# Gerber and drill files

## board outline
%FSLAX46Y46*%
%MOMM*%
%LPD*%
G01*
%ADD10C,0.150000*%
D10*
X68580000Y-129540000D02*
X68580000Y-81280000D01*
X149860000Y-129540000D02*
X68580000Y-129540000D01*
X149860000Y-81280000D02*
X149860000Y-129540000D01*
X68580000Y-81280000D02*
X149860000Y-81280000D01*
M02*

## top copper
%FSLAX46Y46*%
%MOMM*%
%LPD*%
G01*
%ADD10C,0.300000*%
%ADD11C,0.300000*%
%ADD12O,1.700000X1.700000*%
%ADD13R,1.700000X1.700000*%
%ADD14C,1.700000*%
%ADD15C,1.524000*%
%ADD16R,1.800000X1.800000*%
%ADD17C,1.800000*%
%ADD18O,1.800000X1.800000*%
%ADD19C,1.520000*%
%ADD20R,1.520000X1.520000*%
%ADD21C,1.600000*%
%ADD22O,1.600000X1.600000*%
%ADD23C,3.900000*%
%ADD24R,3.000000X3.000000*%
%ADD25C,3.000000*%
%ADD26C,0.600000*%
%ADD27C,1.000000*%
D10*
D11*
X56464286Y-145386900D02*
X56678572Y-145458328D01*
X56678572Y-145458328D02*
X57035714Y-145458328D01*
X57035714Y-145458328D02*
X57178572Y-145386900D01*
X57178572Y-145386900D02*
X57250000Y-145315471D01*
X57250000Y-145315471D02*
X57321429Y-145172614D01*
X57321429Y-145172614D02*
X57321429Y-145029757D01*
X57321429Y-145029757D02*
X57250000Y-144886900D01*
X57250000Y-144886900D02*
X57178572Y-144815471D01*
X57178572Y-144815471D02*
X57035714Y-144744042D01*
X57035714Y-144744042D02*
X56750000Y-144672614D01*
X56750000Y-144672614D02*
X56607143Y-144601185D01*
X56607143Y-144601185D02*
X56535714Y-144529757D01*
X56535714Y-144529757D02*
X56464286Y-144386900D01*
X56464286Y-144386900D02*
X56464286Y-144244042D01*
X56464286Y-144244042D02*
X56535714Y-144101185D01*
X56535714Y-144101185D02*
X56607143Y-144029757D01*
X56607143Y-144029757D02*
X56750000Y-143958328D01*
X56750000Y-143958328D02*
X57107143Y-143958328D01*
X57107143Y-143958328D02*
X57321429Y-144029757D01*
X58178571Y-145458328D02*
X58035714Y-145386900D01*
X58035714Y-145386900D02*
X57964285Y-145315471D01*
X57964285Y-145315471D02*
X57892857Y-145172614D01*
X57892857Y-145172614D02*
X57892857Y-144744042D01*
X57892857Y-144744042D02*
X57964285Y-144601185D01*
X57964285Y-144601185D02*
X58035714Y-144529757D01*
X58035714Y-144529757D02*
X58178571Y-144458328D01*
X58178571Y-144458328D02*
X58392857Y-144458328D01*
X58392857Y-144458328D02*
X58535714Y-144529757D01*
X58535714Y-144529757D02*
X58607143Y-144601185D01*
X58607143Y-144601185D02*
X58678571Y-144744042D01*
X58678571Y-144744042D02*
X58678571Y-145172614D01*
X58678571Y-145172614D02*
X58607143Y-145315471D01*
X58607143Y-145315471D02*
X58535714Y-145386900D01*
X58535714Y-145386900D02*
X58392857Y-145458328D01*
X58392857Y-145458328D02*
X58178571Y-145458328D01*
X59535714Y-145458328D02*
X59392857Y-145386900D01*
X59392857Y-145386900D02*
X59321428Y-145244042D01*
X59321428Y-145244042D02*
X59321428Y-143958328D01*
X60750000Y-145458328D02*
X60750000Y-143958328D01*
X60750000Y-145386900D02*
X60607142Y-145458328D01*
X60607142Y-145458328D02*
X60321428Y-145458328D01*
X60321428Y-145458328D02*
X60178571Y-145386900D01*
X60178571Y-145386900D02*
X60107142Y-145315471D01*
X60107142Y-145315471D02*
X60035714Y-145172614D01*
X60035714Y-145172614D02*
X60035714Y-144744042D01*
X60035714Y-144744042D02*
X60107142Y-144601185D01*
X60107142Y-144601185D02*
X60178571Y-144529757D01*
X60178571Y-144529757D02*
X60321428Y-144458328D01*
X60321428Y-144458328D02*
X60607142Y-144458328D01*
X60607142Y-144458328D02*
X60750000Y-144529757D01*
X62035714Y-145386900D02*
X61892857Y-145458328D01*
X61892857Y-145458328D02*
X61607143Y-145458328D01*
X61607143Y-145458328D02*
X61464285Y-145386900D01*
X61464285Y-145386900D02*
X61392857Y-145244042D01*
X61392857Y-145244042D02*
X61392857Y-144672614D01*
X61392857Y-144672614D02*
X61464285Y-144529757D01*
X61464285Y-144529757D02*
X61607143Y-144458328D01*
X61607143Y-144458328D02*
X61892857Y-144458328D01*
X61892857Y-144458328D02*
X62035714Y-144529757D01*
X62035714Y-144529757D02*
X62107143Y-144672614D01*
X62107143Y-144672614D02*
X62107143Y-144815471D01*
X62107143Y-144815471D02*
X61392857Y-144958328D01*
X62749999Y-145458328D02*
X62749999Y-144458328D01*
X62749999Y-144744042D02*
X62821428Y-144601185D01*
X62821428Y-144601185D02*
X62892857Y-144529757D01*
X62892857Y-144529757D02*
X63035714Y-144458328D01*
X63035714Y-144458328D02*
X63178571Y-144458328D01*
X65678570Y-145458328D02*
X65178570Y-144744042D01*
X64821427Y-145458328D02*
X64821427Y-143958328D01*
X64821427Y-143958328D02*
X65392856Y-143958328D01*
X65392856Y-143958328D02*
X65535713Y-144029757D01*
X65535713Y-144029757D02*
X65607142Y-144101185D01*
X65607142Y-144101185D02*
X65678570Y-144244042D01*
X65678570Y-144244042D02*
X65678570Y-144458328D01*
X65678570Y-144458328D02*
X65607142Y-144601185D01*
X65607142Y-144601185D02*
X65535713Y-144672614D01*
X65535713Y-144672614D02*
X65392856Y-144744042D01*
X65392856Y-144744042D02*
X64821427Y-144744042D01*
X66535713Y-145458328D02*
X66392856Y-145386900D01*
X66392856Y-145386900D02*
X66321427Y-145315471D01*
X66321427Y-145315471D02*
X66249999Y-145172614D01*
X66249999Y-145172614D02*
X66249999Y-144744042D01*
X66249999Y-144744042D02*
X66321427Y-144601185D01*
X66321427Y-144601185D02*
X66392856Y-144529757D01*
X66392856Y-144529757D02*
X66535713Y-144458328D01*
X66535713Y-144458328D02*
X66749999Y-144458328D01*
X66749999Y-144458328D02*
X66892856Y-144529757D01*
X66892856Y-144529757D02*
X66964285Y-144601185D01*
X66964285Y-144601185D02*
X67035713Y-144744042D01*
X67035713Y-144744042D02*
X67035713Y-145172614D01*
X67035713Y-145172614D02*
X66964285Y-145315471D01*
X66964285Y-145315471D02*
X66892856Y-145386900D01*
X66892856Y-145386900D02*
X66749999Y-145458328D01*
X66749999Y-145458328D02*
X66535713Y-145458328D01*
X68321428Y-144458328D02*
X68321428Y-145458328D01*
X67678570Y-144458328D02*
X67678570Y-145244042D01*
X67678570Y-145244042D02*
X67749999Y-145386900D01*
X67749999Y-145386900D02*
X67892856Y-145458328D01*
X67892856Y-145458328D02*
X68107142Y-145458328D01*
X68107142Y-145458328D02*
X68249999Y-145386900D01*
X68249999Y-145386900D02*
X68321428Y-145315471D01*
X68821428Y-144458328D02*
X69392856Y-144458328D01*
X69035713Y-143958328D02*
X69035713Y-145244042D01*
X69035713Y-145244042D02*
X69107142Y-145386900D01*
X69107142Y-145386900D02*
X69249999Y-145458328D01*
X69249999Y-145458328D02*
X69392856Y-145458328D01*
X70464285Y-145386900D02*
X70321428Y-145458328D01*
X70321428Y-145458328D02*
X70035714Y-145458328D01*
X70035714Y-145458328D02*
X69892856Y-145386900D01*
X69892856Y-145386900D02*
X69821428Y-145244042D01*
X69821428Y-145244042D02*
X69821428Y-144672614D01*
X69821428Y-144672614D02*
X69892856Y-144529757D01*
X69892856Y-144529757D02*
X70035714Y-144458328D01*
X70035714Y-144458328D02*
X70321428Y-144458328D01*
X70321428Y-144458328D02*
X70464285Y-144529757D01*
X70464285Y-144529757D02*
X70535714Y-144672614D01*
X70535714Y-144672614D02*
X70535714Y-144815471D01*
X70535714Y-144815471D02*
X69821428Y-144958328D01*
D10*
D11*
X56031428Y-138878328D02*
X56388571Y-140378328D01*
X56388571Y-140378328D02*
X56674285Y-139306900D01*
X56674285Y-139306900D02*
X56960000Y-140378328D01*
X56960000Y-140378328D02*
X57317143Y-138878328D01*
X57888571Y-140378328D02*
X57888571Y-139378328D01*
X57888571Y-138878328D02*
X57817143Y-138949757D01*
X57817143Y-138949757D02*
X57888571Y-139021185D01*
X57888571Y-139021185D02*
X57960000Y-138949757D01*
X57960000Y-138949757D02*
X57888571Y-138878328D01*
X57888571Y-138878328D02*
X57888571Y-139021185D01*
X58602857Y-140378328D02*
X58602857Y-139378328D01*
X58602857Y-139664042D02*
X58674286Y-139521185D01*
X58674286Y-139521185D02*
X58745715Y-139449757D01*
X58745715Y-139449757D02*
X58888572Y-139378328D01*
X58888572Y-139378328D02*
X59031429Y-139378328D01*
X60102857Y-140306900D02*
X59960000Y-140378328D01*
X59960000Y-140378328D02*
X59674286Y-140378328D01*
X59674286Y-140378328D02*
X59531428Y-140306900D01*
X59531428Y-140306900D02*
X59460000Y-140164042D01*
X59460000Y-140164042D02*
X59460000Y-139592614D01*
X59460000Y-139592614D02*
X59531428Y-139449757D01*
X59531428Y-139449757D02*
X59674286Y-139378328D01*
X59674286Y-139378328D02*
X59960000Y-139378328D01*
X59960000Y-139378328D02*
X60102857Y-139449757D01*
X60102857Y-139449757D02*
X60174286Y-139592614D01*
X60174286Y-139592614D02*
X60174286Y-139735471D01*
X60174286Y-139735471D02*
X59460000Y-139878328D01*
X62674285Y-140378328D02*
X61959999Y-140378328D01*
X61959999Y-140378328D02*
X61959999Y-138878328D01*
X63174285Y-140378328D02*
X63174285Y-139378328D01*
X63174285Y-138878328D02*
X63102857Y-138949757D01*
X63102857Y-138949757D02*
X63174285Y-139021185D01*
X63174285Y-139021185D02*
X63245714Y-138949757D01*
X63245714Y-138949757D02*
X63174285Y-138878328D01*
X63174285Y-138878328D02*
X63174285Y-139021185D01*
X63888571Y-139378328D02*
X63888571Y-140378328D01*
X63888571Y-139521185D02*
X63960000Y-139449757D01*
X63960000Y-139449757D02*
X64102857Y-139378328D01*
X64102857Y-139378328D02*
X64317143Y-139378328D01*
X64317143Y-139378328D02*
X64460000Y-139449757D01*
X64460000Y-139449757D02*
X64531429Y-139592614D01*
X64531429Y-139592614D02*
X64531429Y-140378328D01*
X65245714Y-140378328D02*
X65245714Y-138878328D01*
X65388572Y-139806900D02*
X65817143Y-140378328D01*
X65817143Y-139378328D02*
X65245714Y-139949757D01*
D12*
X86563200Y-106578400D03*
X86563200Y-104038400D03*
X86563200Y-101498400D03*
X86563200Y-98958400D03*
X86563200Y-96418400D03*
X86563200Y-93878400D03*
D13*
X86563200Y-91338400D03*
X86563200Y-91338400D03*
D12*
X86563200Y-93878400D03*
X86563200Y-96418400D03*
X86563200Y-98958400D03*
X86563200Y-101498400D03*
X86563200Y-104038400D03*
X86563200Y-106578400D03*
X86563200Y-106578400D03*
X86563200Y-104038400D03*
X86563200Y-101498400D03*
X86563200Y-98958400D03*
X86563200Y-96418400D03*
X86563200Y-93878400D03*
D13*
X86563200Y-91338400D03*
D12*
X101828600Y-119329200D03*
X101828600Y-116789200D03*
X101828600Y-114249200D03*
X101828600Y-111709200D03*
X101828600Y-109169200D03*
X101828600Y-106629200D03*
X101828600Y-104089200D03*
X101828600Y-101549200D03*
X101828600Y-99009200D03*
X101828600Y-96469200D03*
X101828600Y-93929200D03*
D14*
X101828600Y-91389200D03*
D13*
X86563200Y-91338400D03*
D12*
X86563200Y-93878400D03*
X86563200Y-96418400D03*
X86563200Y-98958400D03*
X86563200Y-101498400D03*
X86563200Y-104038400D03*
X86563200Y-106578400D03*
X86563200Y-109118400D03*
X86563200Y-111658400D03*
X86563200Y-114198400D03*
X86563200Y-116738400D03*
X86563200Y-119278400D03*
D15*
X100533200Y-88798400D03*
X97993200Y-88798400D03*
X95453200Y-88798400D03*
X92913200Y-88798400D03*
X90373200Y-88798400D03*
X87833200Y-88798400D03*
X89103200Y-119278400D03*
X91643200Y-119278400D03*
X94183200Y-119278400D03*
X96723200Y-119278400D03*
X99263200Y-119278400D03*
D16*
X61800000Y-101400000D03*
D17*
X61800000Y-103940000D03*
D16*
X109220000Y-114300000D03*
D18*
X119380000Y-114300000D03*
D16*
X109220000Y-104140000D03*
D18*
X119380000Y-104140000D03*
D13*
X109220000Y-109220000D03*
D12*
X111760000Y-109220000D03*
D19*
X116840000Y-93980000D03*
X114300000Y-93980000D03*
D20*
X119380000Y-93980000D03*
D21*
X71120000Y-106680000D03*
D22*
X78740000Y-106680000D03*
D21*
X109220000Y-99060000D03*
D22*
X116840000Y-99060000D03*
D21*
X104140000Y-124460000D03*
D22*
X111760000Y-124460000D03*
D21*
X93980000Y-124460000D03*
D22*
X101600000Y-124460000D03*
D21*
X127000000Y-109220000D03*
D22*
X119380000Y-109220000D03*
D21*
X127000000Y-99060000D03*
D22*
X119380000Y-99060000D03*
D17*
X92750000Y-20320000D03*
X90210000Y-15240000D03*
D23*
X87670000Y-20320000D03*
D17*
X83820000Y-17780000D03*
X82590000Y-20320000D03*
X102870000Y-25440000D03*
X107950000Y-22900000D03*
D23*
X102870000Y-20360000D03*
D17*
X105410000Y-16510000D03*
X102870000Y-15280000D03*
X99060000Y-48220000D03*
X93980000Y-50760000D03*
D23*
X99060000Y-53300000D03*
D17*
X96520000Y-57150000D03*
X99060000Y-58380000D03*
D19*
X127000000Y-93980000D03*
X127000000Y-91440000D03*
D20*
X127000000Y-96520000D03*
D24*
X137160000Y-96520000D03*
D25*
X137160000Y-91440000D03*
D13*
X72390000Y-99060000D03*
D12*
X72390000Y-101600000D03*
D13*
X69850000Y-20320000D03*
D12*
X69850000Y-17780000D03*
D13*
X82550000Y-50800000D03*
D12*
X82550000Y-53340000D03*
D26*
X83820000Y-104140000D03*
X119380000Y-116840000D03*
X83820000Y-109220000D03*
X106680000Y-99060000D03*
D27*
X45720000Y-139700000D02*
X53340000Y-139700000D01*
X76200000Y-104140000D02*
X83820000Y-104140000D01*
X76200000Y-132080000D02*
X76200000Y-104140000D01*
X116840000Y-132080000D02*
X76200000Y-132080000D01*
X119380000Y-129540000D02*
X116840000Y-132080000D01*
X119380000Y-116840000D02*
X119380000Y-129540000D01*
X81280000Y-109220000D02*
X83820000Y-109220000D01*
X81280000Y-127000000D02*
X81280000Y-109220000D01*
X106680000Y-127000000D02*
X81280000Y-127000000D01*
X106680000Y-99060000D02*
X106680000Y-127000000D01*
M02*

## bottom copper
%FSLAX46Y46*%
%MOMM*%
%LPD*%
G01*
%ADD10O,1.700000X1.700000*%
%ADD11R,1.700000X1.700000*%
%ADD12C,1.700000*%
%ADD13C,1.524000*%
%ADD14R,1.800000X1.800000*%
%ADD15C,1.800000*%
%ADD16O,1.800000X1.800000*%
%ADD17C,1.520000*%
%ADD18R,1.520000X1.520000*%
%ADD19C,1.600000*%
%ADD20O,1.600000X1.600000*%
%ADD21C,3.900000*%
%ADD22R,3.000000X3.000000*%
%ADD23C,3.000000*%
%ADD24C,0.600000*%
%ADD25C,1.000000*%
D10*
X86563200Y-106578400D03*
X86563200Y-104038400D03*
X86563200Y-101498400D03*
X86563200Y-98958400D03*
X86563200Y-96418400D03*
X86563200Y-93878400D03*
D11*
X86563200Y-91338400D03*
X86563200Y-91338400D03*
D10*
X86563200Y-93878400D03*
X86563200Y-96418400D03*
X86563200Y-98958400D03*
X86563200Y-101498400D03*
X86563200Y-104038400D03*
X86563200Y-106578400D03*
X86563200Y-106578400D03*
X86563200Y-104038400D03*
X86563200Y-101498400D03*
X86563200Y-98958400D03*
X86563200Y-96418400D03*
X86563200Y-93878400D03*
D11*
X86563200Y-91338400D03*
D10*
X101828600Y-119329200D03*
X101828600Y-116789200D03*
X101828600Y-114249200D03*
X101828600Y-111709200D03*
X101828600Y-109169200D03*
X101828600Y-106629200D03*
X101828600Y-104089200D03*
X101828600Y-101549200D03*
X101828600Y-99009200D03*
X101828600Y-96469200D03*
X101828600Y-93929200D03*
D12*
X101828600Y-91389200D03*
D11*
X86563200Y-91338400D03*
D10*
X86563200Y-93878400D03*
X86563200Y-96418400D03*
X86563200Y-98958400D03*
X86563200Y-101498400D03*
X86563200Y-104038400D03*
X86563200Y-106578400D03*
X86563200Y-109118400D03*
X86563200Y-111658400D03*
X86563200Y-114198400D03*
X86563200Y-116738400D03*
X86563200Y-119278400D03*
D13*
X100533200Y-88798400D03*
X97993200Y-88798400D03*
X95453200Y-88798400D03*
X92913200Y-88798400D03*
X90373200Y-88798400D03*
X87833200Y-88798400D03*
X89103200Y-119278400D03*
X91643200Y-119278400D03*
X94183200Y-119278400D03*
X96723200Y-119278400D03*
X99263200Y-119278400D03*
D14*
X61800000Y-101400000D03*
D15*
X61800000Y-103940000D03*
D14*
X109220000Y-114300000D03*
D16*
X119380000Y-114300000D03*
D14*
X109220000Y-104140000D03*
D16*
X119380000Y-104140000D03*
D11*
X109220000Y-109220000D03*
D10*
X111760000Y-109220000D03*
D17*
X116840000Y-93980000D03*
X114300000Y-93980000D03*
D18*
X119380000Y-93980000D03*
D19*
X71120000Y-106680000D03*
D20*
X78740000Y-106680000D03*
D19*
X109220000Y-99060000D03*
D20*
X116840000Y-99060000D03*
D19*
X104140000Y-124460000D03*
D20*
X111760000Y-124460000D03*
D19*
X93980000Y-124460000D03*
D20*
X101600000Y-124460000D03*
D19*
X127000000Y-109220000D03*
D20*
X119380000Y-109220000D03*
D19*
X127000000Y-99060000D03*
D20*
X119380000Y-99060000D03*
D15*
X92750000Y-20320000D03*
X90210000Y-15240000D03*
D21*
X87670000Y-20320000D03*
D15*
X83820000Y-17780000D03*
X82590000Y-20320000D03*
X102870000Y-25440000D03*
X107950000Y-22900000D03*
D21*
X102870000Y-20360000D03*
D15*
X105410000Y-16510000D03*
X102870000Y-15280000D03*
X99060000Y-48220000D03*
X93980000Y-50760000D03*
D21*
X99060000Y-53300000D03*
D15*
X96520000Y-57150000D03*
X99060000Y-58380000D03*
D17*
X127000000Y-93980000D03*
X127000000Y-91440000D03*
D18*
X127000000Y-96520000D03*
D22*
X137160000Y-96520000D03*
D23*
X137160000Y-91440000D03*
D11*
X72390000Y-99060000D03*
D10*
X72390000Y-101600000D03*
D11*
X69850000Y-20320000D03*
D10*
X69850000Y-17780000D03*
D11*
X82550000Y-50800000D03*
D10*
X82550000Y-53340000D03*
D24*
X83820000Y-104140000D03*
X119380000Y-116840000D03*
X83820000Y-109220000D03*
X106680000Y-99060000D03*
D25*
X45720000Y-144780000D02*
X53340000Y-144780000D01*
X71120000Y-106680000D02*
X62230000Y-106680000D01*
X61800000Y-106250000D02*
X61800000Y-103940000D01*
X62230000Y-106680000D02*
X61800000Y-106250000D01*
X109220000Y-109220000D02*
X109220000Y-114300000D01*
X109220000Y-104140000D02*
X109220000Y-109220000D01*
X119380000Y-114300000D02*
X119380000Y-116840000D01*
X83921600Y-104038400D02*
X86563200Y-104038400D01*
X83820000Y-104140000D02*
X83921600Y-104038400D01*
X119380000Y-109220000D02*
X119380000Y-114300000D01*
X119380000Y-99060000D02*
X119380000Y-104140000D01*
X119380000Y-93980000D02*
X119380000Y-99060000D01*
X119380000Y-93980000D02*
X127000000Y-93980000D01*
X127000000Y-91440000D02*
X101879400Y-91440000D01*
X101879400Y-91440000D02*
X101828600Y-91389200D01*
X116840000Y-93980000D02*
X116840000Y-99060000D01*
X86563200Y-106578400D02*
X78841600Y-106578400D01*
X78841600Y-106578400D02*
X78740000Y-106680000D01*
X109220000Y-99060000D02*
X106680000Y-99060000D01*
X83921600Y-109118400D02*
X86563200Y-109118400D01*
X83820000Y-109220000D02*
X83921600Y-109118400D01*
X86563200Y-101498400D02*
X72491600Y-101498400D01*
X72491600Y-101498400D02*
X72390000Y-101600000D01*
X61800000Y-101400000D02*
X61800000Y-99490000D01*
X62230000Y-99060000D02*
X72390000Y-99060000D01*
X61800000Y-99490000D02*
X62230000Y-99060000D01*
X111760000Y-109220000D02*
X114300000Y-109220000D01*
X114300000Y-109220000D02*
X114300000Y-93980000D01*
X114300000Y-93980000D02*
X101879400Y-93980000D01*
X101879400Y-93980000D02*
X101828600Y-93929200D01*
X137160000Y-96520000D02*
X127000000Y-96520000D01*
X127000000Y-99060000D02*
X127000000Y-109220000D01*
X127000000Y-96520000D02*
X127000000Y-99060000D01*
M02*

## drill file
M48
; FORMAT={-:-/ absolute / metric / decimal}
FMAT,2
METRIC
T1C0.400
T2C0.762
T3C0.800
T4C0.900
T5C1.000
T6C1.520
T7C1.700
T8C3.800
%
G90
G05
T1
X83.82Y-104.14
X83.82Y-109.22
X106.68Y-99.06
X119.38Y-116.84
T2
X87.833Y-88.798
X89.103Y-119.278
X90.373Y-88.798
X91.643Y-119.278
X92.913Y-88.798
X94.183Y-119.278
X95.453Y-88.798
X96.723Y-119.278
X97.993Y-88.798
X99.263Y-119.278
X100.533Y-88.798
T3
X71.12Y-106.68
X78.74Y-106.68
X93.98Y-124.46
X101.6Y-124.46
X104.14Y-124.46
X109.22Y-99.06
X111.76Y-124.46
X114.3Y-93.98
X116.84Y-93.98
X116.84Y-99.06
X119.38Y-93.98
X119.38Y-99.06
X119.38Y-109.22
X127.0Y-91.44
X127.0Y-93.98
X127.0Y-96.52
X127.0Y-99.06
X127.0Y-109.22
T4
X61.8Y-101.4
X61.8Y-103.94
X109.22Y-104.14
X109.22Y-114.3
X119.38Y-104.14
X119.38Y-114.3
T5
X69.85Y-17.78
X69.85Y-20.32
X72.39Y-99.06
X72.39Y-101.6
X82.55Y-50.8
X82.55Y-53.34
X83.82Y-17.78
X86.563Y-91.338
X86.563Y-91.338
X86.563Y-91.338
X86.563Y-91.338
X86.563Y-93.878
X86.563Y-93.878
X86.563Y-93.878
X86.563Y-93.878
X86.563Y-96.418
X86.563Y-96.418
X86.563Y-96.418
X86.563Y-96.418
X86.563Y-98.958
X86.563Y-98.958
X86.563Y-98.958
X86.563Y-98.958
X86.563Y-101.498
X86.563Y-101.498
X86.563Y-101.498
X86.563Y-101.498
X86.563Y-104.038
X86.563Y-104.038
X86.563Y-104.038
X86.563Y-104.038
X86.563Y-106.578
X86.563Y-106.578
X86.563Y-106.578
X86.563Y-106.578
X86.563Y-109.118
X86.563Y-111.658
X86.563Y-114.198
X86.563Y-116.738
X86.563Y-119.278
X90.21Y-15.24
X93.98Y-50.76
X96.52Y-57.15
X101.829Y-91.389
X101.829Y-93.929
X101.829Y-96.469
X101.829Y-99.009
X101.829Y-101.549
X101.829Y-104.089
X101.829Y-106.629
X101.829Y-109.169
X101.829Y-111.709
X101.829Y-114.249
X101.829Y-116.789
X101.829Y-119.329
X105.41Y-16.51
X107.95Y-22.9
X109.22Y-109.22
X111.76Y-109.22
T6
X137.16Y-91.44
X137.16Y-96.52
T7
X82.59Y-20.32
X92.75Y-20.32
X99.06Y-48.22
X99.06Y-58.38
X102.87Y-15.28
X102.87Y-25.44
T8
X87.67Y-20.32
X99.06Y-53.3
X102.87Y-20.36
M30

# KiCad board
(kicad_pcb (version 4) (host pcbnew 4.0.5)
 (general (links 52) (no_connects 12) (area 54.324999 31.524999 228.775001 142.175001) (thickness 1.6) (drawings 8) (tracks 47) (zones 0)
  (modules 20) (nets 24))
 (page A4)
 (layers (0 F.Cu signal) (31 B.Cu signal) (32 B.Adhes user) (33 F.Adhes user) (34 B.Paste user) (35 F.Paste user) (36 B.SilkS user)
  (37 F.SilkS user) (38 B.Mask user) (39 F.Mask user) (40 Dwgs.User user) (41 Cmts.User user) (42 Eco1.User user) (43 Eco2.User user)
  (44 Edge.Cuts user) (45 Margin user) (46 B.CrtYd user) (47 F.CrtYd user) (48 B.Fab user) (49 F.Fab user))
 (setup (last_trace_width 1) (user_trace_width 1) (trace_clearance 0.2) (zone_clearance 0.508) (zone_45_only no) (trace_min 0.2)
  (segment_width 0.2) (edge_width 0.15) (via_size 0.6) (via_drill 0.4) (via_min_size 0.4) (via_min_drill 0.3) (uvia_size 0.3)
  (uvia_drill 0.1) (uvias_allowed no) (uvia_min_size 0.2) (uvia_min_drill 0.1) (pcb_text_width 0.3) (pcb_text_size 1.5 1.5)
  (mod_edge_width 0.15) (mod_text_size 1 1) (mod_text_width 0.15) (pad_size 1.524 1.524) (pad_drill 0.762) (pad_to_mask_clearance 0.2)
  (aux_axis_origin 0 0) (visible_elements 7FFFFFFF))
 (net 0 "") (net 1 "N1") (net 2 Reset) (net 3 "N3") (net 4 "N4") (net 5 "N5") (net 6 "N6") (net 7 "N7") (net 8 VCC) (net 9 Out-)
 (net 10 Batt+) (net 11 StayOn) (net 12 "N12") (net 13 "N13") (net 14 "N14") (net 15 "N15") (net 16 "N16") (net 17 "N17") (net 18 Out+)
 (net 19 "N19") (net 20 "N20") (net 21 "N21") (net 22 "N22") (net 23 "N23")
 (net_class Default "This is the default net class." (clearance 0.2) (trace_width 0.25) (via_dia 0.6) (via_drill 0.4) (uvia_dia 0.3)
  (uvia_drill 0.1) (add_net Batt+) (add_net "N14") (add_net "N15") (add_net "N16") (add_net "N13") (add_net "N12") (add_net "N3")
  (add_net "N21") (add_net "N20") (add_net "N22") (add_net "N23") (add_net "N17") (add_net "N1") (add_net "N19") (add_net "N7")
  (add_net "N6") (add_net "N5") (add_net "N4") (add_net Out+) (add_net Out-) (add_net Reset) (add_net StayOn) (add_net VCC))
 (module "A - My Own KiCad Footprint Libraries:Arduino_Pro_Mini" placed (layer F.Cu) (at 93.98 101.6)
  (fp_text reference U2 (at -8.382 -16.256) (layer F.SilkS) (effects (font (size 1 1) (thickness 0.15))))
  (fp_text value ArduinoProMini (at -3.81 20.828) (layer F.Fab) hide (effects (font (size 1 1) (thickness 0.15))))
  (pad 7 thru_hole oval (at -7.4168 4.9784) (size 1.7 1.7) (drill 1) (layers *.Mask B.Cu) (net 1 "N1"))
  (pad 6 thru_hole oval (at -7.4168 2.4384) (size 1.7 1.7) (drill 1) (layers *.Mask B.Cu) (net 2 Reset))
  (pad 5 thru_hole oval (at -7.4168 -0.1016) (size 1.7 1.7) (drill 1) (layers *.Mask B.Cu) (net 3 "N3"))
  (pad 4 thru_hole oval (at -7.4168 -2.6416) (size 1.7 1.7) (drill 1) (layers *.Mask B.Cu) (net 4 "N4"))
  (pad 3 thru_hole oval (at -7.4168 -5.1816) (size 1.7 1.7) (drill 1) (layers *.Mask B.Cu) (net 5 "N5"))
  (pad 2 thru_hole oval (at -7.4168 -7.7216) (size 1.7 1.7) (drill 1) (layers *.Mask B.Cu) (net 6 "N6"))
  (pad 1 thru_hole rect (at -7.4168 -10.2616) (size 1.7 1.7) (drill 1) (layers *.Mask B.Cu) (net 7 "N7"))
  (pad 1 thru_hole rect (at -7.4168 -10.2616) (size 1.7 1.7) (drill 1) (layers *.Mask B.Cu) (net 7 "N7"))
  (pad 2 thru_hole oval (at -7.4168 -7.7216) (size 1.7 1.7) (drill 1) (layers *.Mask B.Cu) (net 6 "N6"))
  (pad 3 thru_hole oval (at -7.4168 -5.1816) (size 1.7 1.7) (drill 1) (layers *.Mask B.Cu) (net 5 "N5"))
  (pad 4 thru_hole oval (at -7.4168 -2.6416) (size 1.7 1.7) (drill 1) (layers *.Mask B.Cu) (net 4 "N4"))
  (pad 5 thru_hole oval (at -7.4168 -0.1016) (size 1.7 1.7) (drill 1) (layers *.Mask B.Cu) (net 3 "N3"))
  (pad 6 thru_hole oval (at -7.4168 2.4384) (size 1.7 1.7) (drill 1) (layers *.Mask B.Cu) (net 2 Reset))
  (pad 7 thru_hole oval (at -7.4168 4.9784) (size 1.7 1.7) (drill 1) (layers *.Mask B.Cu) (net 1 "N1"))
  (pad 7 thru_hole oval (at -7.4168 4.9784) (size 1.7 1.7) (drill 1) (layers *.Mask B.Cu) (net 1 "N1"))
  (pad 6 thru_hole oval (at -7.4168 2.4384) (size 1.7 1.7) (drill 1) (layers *.Mask B.Cu) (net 2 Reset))
  (pad 5 thru_hole oval (at -7.4168 -0.1016) (size 1.7 1.7) (drill 1) (layers *.Mask B.Cu) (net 3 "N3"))
  (pad 4 thru_hole oval (at -7.4168 -2.6416) (size 1.7 1.7) (drill 1) (layers *.Mask B.Cu) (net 4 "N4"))
  (pad 3 thru_hole oval (at -7.4168 -5.1816) (size 1.7 1.7) (drill 1) (layers *.Mask B.Cu) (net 5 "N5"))
  (pad 2 thru_hole oval (at -7.4168 -7.7216) (size 1.7 1.7) (drill 1) (layers *.Mask B.Cu) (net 6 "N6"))
  (pad 1 thru_hole rect (at -7.4168 -10.2616) (size 1.7 1.7) (drill 1) (layers *.Mask B.Cu) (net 7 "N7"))
  (pad 18 thru_hole oval (at 7.8486 17.7292) (size 1.7 1.7) (drill 1) (layers *.Mask B.Cu))
  (pad 19 thru_hole oval (at 7.8486 15.1892) (size 1.7 1.7) (drill 1) (layers *.Mask B.Cu))
  (pad 20 thru_hole oval (at 7.8486 12.6492) (size 1.7 1.7) (drill 1) (layers *.Mask B.Cu))
  (pad 21 thru_hole oval (at 7.8486 10.1092) (size 1.7 1.7) (drill 1) (layers *.Mask B.Cu))
  (pad 22 thru_hole oval (at 7.8486 7.5692) (size 1.7 1.7) (drill 1) (layers *.Mask B.Cu))
  (pad 23 thru_hole oval (at 7.8486 5.0292) (size 1.7 1.7) (drill 1) (layers *.Mask B.Cu))
  (pad 24 thru_hole oval (at 7.8486 2.4892) (size 1.7 1.7) (drill 1) (layers *.Mask B.Cu))
  (pad 25 thru_hole oval (at 7.8486 -0.0508) (size 1.7 1.7) (drill 1) (layers *.Mask B.Cu))
  (pad 26 thru_hole oval (at 7.8486 -2.5908) (size 1.7 1.7) (drill 1) (layers *.Mask B.Cu) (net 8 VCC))
  (pad 27 thru_hole oval (at 7.8486 -5.1308) (size 1.7 1.7) (drill 1) (layers *.Mask B.Cu))
  (pad 28 thru_hole oval (at 7.8486 -7.6708) (size 1.7 1.7) (drill 1) (layers *.Mask B.Cu) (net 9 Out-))
  (pad 29 thru_hole circle (at 7.8486 -10.2108) (size 1.7 1.7) (drill 1) (layers *.Mask B.Cu) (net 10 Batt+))
  (pad 1 thru_hole rect (at -7.4168 -10.2616) (size 1.7 1.7) (drill 1) (layers *.Mask B.Cu) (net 7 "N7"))
  (pad 2 thru_hole oval (at -7.4168 -7.7216) (size 1.7 1.7) (drill 1) (layers *.Mask B.Cu) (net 6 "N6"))
  (pad 3 thru_hole oval (at -7.4168 -5.1816) (size 1.7 1.7) (drill 1) (layers *.Mask B.Cu) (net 5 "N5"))
  (pad 4 thru_hole oval (at -7.4168 -2.6416) (size 1.7 1.7) (drill 1) (layers *.Mask B.Cu) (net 4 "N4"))
  (pad 5 thru_hole oval (at -7.4168 -0.1016) (size 1.7 1.7) (drill 1) (layers *.Mask B.Cu) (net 3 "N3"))
  (pad 6 thru_hole oval (at -7.4168 2.4384) (size 1.7 1.7) (drill 1) (layers *.Mask B.Cu) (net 2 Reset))
  (pad 7 thru_hole oval (at -7.4168 4.9784) (size 1.7 1.7) (drill 1) (layers *.Mask B.Cu) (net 1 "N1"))
  (pad 8 thru_hole oval (at -7.4168 7.5184) (size 1.7 1.7) (drill 1) (layers *.Mask B.Cu) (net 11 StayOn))
  (pad 9 thru_hole oval (at -7.4168 10.0584) (size 1.7 1.7) (drill 1) (layers *.Mask B.Cu))
  (pad 10 thru_hole oval (at -7.4168 12.5984) (size 1.7 1.7) (drill 1) (layers *.Mask B.Cu))
  (pad 11 thru_hole oval (at -7.4168 15.1384) (size 1.7 1.7) (drill 1) (layers *.Mask B.Cu))
  (pad 12 thru_hole oval (at -7.4168 17.6784) (size 1.7 1.7) (drill 1) (layers *.Mask B.Cu))
  (pad 30 thru_hole circle (at 6.5532 -12.8016) (size 1.524 1.524) (drill 0.762) (layers *.Mask F.Cu))
  (pad 31 thru_hole circle (at 4.0132 -12.8016) (size 1.524 1.524) (drill 0.762) (layers *.Mask F.Cu))
  (pad 32 thru_hole circle (at 1.4732 -12.8016) (size 1.524 1.524) (drill 0.762) (layers *.Mask F.Cu))
  (pad 33 thru_hole circle (at -1.0668 -12.8016) (size 1.524 1.524) (drill 0.762) (layers *.Mask F.Cu))
  (pad 34 thru_hole circle (at -3.6068 -12.8016) (size 1.524 1.524) (drill 0.762) (layers *.Mask F.Cu))
  (pad 35 thru_hole circle (at -6.1468 -12.8016) (size 1.524 1.524) (drill 0.762) (layers *.Mask F.Cu))
  (pad 13 thru_hole circle (at -4.8768 17.6784) (size 1.524 1.524) (drill 0.762) (layers *.Mask F.Cu) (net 9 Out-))
  (pad 14 thru_hole circle (at -2.3368 17.6784) (size 1.524 1.524) (drill 0.762) (layers *.Mask F.Cu) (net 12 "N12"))
  (pad 15 thru_hole circle (at 0.2032 17.6784) (size 1.524 1.524) (drill 0.762) (layers *.Mask F.Cu) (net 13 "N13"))
  (pad 16 thru_hole circle (at 2.7432 17.6784) (size 1.524 1.524) (drill 0.762) (layers *.Mask F.Cu))
  (pad 17] thru_hole circle (at 5.2832 17.6784) (size 1.524 1.524) (drill 0.762) (layers *.Mask F.Cu)))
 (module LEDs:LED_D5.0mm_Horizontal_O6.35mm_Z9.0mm (layer F.Cu) (at 61.8 101.4 270)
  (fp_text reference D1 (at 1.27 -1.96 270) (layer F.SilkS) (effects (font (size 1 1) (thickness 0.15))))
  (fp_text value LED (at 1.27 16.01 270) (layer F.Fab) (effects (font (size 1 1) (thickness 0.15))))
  (pad 1 thru_hole rect (at 0 0 270) (size 1.8 1.8) (drill 0.9) (layers *.Cu *.Mask) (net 9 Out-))
  (pad 2 thru_hole circle (at 2.54 0 270) (size 1.8 1.8) (drill 0.9) (layers *.Cu *.Mask) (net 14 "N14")))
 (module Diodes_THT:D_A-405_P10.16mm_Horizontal (layer F.Cu) (at 109.22 114.3)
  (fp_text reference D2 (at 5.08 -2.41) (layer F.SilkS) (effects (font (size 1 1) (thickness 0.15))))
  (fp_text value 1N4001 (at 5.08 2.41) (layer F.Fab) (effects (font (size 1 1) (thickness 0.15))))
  (pad 1 thru_hole rect (at 0 0) (size 1.8 1.8) (drill 0.9) (layers *.Cu *.Mask) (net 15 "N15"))
  (pad 2 thru_hole oval (at 10.16 0) (size 1.8 1.8) (drill 0.9) (layers *.Cu *.Mask) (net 2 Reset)))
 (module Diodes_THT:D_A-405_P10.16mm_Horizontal (layer F.Cu) (at 109.22 104.14)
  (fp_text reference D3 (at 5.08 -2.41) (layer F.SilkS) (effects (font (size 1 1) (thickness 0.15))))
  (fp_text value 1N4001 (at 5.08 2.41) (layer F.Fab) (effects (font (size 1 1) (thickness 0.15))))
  (pad 1 thru_hole rect (at 0 0) (size 1.8 1.8) (drill 0.9) (layers *.Cu *.Mask) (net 15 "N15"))
  (pad 2 thru_hole oval (at 10.16 0) (size 1.8 1.8) (drill 0.9) (layers *.Cu *.Mask) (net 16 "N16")))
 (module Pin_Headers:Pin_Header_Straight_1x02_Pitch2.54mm (layer F.Cu) (at 109.22 109.22 90)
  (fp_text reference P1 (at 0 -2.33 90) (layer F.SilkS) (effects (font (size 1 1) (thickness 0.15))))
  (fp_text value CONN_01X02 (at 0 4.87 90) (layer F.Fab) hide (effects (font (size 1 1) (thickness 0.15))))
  (pad 1 thru_hole rect (at 0 0 90) (size 1.7 1.7) (drill 1) (layers *.Cu *.Mask) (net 15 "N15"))
  (pad 2 thru_hole oval (at 0 2.54 90) (size 1.7 1.7) (drill 1) (layers *.Cu *.Mask) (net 9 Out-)))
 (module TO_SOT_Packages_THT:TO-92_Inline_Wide (layer F.Cu) (at 119.38 93.98 180)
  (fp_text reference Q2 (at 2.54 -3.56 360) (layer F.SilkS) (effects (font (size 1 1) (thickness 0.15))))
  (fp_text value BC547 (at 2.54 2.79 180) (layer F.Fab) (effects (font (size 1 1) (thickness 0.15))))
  (pad 2 thru_hole circle (at 2.54 0 270) (size 1.52 1.52) (drill 0.8) (layers *.Cu *.Mask) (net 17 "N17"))
  (pad 3 thru_hole circle (at 5.08 0 270) (size 1.52 1.52) (drill 0.8) (layers *.Cu *.Mask) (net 9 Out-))
  (pad 1 thru_hole rect (at 0 0 270) (size 1.52 1.52) (drill 0.8) (layers *.Cu *.Mask) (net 16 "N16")))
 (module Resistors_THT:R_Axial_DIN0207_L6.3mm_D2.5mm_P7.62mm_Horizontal (layer F.Cu) (at 71.12 106.68)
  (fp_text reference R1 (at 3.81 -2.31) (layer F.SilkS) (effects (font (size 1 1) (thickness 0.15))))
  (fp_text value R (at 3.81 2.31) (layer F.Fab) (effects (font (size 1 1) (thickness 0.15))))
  (pad 1 thru_hole circle (at 0 0) (size 1.6 1.6) (drill 0.8) (layers *.Cu *.Mask) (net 14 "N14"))
  (pad 2 thru_hole oval (at 7.62 0) (size 1.6 1.6) (drill 0.8) (layers *.Cu *.Mask) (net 1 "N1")))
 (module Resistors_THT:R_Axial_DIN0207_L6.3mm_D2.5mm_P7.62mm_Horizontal (layer F.Cu) (at 109.22 99.06)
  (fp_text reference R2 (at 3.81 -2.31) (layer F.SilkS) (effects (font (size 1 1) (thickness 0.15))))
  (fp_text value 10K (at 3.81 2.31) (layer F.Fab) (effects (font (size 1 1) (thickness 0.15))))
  (pad 1 thru_hole circle (at 0 0) (size 1.6 1.6) (drill 0.8) (layers *.Cu *.Mask) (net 11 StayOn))
  (pad 2 thru_hole oval (at 7.62 0) (size 1.6 1.6) (drill 0.8) (layers *.Cu *.Mask) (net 17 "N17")))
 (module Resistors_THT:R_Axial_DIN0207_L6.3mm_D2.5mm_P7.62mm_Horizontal (layer F.Cu) (at 104.14 124.46)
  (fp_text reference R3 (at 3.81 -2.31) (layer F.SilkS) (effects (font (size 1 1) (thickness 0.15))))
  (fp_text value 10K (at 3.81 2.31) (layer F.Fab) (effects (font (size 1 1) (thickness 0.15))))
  (pad 1 thru_hole circle (at 0 0) (size 1.6 1.6) (drill 0.8) (layers *.Cu *.Mask) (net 8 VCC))
  (pad 2 thru_hole oval (at 7.62 0) (size 1.6 1.6) (drill 0.8) (layers *.Cu *.Mask) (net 13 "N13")))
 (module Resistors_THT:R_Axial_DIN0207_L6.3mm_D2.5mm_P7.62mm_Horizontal (layer F.Cu) (at 93.98 124.46)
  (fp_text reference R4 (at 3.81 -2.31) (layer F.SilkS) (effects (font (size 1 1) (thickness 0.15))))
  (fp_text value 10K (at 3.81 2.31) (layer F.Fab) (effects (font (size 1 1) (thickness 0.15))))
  (pad 1 thru_hole circle (at 0 0) (size 1.6 1.6) (drill 0.8) (layers *.Cu *.Mask) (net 8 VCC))
  (pad 2 thru_hole oval (at 7.62 0) (size 1.6 1.6) (drill 0.8) (layers *.Cu *.Mask) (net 12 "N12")))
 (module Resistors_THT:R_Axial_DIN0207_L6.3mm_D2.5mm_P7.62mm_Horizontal (layer F.Cu) (at 127 109.22 180)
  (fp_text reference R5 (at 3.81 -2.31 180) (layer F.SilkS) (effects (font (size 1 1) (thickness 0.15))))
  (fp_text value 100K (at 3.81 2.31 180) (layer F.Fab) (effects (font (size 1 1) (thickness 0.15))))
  (pad 1 thru_hole circle (at 0 0 180) (size 1.6 1.6) (drill 0.8) (layers *.Cu *.Mask) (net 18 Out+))
  (pad 2 thru_hole oval (at 7.62 0 180) (size 1.6 1.6) (drill 0.8) (layers *.Cu *.Mask) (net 2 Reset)))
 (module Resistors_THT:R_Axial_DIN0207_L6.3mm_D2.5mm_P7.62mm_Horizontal (layer F.Cu) (at 127 99.06 180)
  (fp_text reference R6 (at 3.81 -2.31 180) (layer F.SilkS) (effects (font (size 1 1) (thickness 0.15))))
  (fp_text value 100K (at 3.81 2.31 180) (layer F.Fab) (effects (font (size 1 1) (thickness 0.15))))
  (pad 1 thru_hole circle (at 0 0 180) (size 1.6 1.6) (drill 0.8) (layers *.Cu *.Mask) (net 18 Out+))
  (pad 2 thru_hole oval (at 7.62 0 180) (size 1.6 1.6) (drill 0.8) (layers *.Cu *.Mask) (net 16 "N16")))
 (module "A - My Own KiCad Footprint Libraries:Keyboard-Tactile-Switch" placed (layer F.Cu) (at 87.63 20.32 270)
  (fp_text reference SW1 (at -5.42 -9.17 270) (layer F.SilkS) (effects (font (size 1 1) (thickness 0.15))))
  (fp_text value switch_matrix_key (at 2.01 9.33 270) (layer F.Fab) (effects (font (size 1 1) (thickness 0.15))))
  (pad 10 thru_hole circle (at 0 -5.12 270) (size 1.8 1.8) (drill 1.7) (layers *.Cu *.Mask))
  (pad 1 thru_hole circle (at -5.08 -2.58 270) (size 1.8 1.8) (drill 1) (layers *.Cu *.Mask) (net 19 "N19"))
  (pad 10 thru_hole circle (at 0 -0.04 270) (size 3.9 3.9) (drill 3.8) (layers *.Cu *.Mask))
  (pad 2 thru_hole circle (at -2.54 3.81 270) (size 1.8 1.8) (drill 1) (layers *.Cu *.Mask) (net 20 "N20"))
  (pad 10 thru_hole circle (at 0 5.04 270) (size 1.8 1.8) (drill 1.7) (layers *.Cu *.Mask)))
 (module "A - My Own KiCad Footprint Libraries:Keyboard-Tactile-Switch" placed (layer F.Cu) (at 102.87 20.32 180)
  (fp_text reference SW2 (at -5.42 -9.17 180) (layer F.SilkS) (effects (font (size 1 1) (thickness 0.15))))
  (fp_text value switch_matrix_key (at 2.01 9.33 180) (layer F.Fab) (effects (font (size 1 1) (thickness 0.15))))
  (pad 10 thru_hole circle (at 0 -5.12 180) (size 1.8 1.8) (drill 1.7) (layers *.Cu *.Mask))
  (pad 1 thru_hole circle (at -5.08 -2.58 180) (size 1.8 1.8) (drill 1) (layers *.Cu *.Mask) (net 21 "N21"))
  (pad 10 thru_hole circle (at 0 -0.04 180) (size 3.9 3.9) (drill 3.8) (layers *.Cu *.Mask))
  (pad 2 thru_hole circle (at -2.54 3.81 180) (size 1.8 1.8) (drill 1) (layers *.Cu *.Mask) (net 19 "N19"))
  (pad 10 thru_hole circle (at 0 5.04 180) (size 1.8 1.8) (drill 1.7) (layers *.Cu *.Mask)))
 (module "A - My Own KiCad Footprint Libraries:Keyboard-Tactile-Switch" (layer F.Cu) (at 99.06 53.34)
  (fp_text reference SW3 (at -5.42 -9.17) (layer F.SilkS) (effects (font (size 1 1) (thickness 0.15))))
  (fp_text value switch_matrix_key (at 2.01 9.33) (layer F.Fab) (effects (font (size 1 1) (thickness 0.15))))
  (pad 10 thru_hole circle (at 0 -5.12) (size 1.8 1.8) (drill 1.7) (layers *.Cu *.Mask))
  (pad 1 thru_hole circle (at -5.08 -2.58) (size 1.8 1.8) (drill 1) (layers *.Cu *.Mask) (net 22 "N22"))
  (pad 10 thru_hole circle (at 0 -0.04) (size 3.9 3.9) (drill 3.8) (layers *.Cu *.Mask))
  (pad 2 thru_hole circle (at -2.54 3.81) (size 1.8 1.8) (drill 1) (layers *.Cu *.Mask) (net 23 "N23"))
  (pad 10 thru_hole circle (at 0 5.04) (size 1.8 1.8) (drill 1.7) (layers *.Cu *.Mask)))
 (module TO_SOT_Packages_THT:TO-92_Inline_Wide (layer F.Cu) (at 127 96.52 90)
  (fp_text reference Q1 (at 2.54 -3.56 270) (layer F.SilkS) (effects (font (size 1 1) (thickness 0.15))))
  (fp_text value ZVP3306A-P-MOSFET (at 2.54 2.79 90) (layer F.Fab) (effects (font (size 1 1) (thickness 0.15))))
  (pad 2 thru_hole circle (at 2.54 0 180) (size 1.52 1.52) (drill 0.8) (layers *.Cu *.Mask) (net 16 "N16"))
  (pad 3 thru_hole circle (at 5.08 0 180) (size 1.52 1.52) (drill 0.8) (layers *.Cu *.Mask) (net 10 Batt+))
  (pad 1 thru_hole rect (at 0 0 180) (size 1.52 1.52) (drill 0.8) (layers *.Cu *.Mask) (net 18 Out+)))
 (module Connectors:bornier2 (layer F.Cu) (at 137.16 96.52 90)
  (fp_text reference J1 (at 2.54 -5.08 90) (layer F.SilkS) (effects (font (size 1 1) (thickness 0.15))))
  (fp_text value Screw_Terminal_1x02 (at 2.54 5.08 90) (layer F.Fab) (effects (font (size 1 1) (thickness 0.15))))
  (pad 1 thru_hole rect (at 0 0 90) (size 3 3) (drill 1.52) (layers *.Cu *.Mask) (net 18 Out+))
  (pad 2 thru_hole circle (at 5.08 0 90) (size 3 3) (drill 1.52) (layers *.Cu *.Mask) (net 9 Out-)))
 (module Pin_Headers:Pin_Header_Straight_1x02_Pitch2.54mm (layer F.Cu) (at 72.39 99.06)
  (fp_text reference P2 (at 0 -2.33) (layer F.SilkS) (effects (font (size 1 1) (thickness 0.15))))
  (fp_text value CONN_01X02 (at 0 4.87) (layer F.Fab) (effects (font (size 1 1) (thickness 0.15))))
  (pad 1 thru_hole rect (at 0 0) (size 1.7 1.7) (drill 1) (layers *.Cu *.Mask) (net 9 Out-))
  (pad 2 thru_hole oval (at 0 2.54) (size 1.7 1.7) (drill 1) (layers *.Cu *.Mask) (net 3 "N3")))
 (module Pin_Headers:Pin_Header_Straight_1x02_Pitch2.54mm (layer F.Cu) (at 69.85 20.32 180)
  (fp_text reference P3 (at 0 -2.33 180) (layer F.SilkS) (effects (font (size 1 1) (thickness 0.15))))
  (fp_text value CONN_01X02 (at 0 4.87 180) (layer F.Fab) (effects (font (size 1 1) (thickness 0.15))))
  (pad 1 thru_hole rect (at 0 0 180) (size 1.7 1.7) (drill 1) (layers *.Cu *.Mask) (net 21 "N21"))
  (pad 2 thru_hole oval (at 0 2.54 180) (size 1.7 1.7) (drill 1) (layers *.Cu *.Mask) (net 20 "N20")))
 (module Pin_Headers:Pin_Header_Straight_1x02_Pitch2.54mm (layer F.Cu) (at 82.55 50.8)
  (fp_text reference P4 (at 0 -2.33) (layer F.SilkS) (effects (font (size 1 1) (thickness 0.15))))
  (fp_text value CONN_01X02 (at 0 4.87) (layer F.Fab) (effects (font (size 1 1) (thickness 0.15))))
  (pad 1 thru_hole rect (at 0 0) (size 1.7 1.7) (drill 1) (layers *.Cu *.Mask) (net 22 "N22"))
  (pad 2 thru_hole oval (at 0 2.54) (size 1.7 1.7) (drill 1) (layers *.Cu *.Mask) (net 23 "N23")))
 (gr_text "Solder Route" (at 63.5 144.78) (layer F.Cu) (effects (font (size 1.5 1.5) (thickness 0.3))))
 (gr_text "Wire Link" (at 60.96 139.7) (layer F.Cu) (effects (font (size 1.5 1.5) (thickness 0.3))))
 (gr_line (start 68.58 129.54) (end 68.58 81.28) (angle 90) (layer Edge.Cuts) (width 0.15))
 (gr_line (start 149.86 129.54) (end 68.58 129.54) (angle 90) (layer Edge.Cuts) (width 0.15))
 (gr_line (start 149.86 81.28) (end 149.86 129.54) (angle 90) (layer Edge.Cuts) (width 0.15))
 (gr_line (start 68.58 81.28) (end 149.86 81.28) (angle 90) (layer Edge.Cuts) (width 0.15))
 (segment (start 45.72 144.78) (end 53.34 144.78) (width 1) (layer B.Cu) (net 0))
 (segment (start 45.72 139.7) (end 53.34 139.7) (width 1) (layer F.Cu) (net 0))
 (segment (start 71.12 106.68) (end 62.23 106.68) (width 1) (layer B.Cu) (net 14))
 (segment (start 61.8 106.25) (end 61.8 103.94) (width 1) (layer B.Cu) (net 14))
 (segment (start 62.23 106.68) (end 61.8 106.25) (width 1) (layer B.Cu) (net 14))
 (segment (start 109.22 109.22) (end 109.22 114.3) (width 1) (layer B.Cu) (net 15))
 (segment (start 109.22 104.14) (end 109.22 109.22) (width 1) (layer B.Cu) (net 15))
 (segment (start 119.38 114.3) (end 119.38 116.84) (width 1) (layer B.Cu) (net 2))
 (segment (start 83.9216 104.0384) (end 86.5632 104.0384) (width 1) (layer B.Cu) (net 2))
 (segment (start 83.82 104.14) (end 83.9216 104.0384) (width 1) (layer B.Cu) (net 2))
 (via (at 83.82 104.14) (size 0.6) (drill 0.4) (layers F.Cu B.Cu) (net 2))
 (segment (start 76.2 104.14) (end 83.82 104.14) (width 1) (layer F.Cu) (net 2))
 (segment (start 76.2 132.08) (end 76.2 104.14) (width 1) (layer F.Cu) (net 2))
 (segment (start 116.84 132.08) (end 76.2 132.08) (width 1) (layer F.Cu) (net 2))
 (segment (start 119.38 129.54) (end 116.84 132.08) (width 1) (layer F.Cu) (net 2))
 (segment (start 119.38 116.84) (end 119.38 129.54) (width 1) (layer F.Cu) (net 2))
 (via (at 119.38 116.84) (size 0.6) (drill 0.4) (layers F.Cu B.Cu) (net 2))
 (segment (start 119.38 109.22) (end 119.38 114.3) (width 1) (layer B.Cu) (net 2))
 (segment (start 119.38 99.06) (end 119.38 104.14) (width 1) (layer B.Cu) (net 16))
 (segment (start 119.38 93.98) (end 119.38 99.06) (width 1) (layer B.Cu) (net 16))
 (segment (start 119.38 93.98) (end 127 93.98) (width 1) (layer B.Cu) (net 16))
 (segment (start 127 91.44) (end 101.8794 91.44) (width 1) (layer B.Cu) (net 10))
 (segment (start 101.8794 91.44) (end 101.8286 91.3892) (width 1) (layer B.Cu) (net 10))
 (segment (start 116.84 93.98) (end 116.84 99.06) (width 1) (layer B.Cu) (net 17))
 (segment (start 86.5632 106.5784) (end 78.8416 106.5784) (width 1) (layer B.Cu) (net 1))
 (segment (start 78.8416 106.5784) (end 78.74 106.68) (width 1) (layer B.Cu) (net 1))
 (segment (start 109.22 99.06) (end 106.68 99.06) (width 1) (layer B.Cu) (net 11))
 (segment (start 83.9216 109.1184) (end 86.5632 109.1184) (width 1) (layer B.Cu) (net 11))
 (segment (start 83.82 109.22) (end 83.9216 109.1184) (width 1) (layer B.Cu) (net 11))
 (via (at 83.82 109.22) (size 0.6) (drill 0.4) (layers F.Cu B.Cu) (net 11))
 (segment (start 81.28 109.22) (end 83.82 109.22) (width 1) (layer F.Cu) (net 11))
 (segment (start 81.28 127) (end 81.28 109.22) (width 1) (layer F.Cu) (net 11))
 (segment (start 106.68 127) (end 81.28 127) (width 1) (layer F.Cu) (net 11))
 (segment (start 106.68 99.06) (end 106.68 127) (width 1) (layer F.Cu) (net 11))
 (via (at 106.68 99.06) (size 0.6) (drill 0.4) (layers F.Cu B.Cu) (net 11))
 (segment (start 86.5632 101.4984) (end 72.4916 101.4984) (width 1) (layer B.Cu) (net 3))
 (segment (start 72.4916 101.4984) (end 72.39 101.6) (width 1) (layer B.Cu) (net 3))
 (segment (start 61.8 101.4) (end 61.8 99.49) (width 1) (layer B.Cu) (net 9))
 (segment (start 62.23 99.06) (end 72.39 99.06) (width 1) (layer B.Cu) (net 9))
 (segment (start 61.8 99.49) (end 62.23 99.06) (width 1) (layer B.Cu) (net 9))
 (segment (start 111.76 109.22) (end 114.3 109.22) (width 1) (layer B.Cu) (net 9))
 (segment (start 114.3 109.22) (end 114.3 93.98) (width 1) (layer B.Cu) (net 9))
 (segment (start 114.3 93.98) (end 101.8794 93.98) (width 1) (layer B.Cu) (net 9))
 (segment (start 101.8794 93.98) (end 101.8286 93.9292) (width 1) (layer B.Cu) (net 9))
 (segment (start 137.16 96.52) (end 127 96.52) (width 1) (layer B.Cu) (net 18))
 (segment (start 127 99.06) (end 127 109.22) (width 1) (layer B.Cu) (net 18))
 (segment (start 127 96.52) (end 127 99.06) (width 1) (layer B.Cu) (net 18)))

